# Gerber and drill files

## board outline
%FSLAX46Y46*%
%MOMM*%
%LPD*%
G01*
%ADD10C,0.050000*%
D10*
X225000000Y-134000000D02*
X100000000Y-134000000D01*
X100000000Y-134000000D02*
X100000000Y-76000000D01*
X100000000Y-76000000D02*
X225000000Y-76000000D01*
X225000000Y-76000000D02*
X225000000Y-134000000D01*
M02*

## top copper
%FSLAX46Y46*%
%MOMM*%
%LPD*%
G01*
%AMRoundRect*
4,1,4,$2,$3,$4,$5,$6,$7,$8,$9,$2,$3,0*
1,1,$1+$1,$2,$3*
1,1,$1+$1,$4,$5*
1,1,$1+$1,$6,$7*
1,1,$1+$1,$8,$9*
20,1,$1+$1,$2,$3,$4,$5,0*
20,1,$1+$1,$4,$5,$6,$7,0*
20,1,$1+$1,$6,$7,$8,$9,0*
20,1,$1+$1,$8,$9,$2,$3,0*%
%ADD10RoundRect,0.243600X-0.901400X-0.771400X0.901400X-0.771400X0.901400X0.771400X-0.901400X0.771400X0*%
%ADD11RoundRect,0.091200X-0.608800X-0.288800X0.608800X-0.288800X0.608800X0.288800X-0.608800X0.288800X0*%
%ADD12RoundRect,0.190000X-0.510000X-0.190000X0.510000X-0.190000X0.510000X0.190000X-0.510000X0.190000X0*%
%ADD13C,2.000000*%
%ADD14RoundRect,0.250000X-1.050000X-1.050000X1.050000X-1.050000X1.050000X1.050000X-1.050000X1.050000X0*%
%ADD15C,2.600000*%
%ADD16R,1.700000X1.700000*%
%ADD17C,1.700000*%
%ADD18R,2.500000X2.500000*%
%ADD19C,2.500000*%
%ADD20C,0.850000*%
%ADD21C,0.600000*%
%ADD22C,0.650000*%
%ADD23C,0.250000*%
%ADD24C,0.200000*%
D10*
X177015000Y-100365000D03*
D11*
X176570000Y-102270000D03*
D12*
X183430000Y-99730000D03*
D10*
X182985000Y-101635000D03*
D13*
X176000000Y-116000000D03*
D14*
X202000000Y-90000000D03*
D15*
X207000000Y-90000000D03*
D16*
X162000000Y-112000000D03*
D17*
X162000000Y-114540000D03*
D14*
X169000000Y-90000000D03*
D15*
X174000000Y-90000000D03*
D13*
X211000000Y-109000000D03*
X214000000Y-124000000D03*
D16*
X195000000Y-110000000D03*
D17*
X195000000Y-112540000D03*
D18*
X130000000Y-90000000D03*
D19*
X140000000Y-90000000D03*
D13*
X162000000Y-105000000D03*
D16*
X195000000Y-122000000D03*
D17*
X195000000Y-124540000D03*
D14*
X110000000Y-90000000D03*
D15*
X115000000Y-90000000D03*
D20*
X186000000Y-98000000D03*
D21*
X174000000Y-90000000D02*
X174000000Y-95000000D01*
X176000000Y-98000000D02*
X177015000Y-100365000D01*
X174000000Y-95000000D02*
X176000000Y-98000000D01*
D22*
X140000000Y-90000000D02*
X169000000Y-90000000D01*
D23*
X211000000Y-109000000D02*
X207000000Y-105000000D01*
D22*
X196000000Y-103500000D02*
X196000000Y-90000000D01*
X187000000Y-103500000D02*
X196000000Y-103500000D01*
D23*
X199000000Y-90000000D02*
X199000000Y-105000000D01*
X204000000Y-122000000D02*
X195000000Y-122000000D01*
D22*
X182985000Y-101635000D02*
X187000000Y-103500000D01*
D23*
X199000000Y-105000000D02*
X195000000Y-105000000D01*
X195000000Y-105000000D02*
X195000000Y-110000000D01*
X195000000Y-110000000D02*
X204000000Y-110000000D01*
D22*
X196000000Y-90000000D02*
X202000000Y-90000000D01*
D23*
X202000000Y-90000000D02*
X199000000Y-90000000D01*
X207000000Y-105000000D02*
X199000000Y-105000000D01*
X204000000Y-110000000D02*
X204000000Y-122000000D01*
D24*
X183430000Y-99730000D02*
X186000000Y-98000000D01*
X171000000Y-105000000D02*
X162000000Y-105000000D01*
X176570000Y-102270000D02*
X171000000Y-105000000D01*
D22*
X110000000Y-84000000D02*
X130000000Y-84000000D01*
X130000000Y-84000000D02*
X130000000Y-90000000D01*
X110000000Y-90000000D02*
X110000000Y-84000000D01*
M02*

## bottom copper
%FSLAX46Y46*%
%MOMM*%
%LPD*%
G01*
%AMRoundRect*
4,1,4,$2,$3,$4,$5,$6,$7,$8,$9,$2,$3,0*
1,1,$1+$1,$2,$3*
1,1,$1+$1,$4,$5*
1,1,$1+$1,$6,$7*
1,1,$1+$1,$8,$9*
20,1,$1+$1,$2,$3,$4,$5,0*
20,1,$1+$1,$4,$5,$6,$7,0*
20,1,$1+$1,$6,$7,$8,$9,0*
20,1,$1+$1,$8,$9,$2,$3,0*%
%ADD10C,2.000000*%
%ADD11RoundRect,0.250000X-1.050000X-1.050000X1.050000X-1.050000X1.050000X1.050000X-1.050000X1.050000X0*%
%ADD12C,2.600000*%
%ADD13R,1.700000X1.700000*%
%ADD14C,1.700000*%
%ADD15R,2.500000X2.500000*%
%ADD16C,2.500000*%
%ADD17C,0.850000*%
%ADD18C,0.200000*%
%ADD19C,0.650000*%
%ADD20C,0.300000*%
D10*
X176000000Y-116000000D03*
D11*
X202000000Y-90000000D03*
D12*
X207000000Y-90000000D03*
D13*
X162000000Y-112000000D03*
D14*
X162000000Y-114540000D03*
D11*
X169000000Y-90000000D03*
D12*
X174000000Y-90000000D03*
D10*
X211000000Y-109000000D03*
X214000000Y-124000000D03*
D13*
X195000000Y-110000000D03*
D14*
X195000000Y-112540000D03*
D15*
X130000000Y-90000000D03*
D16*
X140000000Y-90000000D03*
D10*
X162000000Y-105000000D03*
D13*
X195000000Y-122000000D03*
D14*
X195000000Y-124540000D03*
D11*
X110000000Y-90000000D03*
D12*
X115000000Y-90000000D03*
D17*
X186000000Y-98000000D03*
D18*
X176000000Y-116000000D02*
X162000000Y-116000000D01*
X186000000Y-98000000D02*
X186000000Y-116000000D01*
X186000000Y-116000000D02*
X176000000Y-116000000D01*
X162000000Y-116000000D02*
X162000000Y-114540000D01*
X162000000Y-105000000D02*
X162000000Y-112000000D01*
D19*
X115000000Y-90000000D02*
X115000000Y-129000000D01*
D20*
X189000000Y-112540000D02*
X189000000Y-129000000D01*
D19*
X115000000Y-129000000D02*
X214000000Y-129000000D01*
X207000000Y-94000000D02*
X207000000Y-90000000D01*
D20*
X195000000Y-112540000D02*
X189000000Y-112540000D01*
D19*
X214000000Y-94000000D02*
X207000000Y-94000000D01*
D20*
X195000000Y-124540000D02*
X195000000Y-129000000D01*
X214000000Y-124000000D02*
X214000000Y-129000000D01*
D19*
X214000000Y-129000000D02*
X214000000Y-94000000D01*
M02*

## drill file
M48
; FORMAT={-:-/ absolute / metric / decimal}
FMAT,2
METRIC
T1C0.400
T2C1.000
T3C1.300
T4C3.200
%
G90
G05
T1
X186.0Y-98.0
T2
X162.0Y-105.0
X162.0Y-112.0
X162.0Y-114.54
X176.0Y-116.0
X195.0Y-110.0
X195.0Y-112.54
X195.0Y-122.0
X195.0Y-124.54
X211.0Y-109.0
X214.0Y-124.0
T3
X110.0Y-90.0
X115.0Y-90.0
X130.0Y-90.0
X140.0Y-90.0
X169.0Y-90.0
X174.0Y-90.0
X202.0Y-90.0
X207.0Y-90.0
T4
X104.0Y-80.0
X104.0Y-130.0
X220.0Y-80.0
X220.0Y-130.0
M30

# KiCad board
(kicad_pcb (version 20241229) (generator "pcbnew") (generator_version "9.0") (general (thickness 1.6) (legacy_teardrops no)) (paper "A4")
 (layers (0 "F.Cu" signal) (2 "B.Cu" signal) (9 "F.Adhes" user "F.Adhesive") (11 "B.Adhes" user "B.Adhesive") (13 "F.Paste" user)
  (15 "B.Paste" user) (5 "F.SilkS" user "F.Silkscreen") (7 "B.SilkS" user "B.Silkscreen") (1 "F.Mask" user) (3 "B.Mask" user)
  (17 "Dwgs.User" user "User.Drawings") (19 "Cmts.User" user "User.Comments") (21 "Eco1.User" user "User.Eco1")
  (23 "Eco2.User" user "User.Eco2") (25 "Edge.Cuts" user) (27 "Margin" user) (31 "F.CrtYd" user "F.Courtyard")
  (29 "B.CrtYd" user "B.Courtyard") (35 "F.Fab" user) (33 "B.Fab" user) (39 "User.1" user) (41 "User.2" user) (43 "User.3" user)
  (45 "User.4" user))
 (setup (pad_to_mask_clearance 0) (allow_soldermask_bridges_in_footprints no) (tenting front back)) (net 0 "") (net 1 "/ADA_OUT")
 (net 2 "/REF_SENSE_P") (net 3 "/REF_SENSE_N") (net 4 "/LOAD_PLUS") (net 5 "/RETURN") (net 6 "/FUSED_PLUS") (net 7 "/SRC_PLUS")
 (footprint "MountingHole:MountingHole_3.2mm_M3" (layer "F.Cu") (at 220 130)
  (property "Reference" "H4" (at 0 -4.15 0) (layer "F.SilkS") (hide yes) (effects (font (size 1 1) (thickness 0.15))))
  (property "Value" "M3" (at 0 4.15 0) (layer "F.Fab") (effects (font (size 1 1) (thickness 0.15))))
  (pad "" np_thru_hole circle (at 0 0) (size 3.2 3.2) (drill 3.2) (layers "*.Cu" "*.Mask")))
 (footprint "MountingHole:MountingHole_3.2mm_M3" (layer "F.Cu") (at 104 80)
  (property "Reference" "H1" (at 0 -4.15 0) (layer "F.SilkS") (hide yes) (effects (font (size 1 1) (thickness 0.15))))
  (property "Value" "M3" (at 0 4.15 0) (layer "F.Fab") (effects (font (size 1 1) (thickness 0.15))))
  (pad "" np_thru_hole circle (at 0 0) (size 3.2 3.2) (drill 3.2) (layers "*.Cu" "*.Mask")))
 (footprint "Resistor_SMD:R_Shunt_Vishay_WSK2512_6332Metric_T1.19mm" (layer "F.Cu") (at 180 101)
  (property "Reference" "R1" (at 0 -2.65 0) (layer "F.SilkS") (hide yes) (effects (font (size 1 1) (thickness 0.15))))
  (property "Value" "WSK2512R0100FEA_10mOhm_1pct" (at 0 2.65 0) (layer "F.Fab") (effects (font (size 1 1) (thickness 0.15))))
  (pad "1" smd roundrect (at -2.985 -0.635) (size 2.29 2.03) (layers "F.Cu" "F.Mask" "F.Paste") (roundrect_rratio 0.12) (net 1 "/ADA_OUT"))
  (pad "2" smd roundrect (at -3.43 1.27) (size 1.4 0.76) (layers "F.Cu" "F.Mask" "F.Paste") (roundrect_rratio 0.12) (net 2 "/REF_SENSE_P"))
  (pad "3" smd roundrect (at 3.43 -1.27) (size 1.4 0.76) (layers "F.Cu" "F.Mask" "F.Paste") (roundrect_rratio 0.25) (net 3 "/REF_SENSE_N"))
  (pad "4" smd roundrect (at 2.985 0.635) (size 2.29 2.03) (layers "F.Cu" "F.Mask" "F.Paste") (roundrect_rratio 0.12) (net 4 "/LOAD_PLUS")))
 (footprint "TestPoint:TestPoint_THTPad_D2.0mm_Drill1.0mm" (layer "F.Cu") (at 176 116)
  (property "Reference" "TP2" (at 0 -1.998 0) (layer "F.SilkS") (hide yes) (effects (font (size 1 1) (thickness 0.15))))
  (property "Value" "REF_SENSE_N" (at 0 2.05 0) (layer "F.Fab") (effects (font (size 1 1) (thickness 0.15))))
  (pad "1" thru_hole circle (at 0 0) (size 2 2) (drill 1) (layers "*.Cu" "*.Mask") (remove_unused_layers no) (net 3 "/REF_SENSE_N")))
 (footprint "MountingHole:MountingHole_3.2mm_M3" (layer "F.Cu") (at 220 80)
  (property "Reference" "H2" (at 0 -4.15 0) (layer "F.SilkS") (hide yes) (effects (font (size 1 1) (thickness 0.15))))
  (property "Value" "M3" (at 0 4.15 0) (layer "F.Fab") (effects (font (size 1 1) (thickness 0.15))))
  (pad "" np_thru_hole circle (at 0 0) (size 3.2 3.2) (drill 3.2) (layers "*.Cu" "*.Mask")))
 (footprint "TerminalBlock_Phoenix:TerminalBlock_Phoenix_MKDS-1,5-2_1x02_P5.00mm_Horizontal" (layer "F.Cu") (at 202 90)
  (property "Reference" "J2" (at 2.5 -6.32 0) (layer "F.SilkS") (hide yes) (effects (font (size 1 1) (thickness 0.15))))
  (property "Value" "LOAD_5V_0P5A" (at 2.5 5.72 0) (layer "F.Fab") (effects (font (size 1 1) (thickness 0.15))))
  (pad "1" thru_hole roundrect (at 0 0) (size 2.6 2.6) (drill 1.3) (layers "*.Cu" "*.Mask") (remove_unused_layers no)
   (roundrect_rratio 0.096154) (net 4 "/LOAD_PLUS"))
  (pad "2" thru_hole circle (at 5 0) (size 2.6 2.6) (drill 1.3) (layers "*.Cu" "*.Mask") (remove_unused_layers no) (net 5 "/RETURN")))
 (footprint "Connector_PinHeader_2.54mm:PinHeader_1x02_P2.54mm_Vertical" (layer "F.Cu") (at 162 112)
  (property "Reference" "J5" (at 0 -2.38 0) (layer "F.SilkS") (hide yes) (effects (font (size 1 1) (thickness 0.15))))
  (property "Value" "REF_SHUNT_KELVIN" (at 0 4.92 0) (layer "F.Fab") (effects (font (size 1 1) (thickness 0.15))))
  (pad "1" thru_hole rect (at 0 0) (size 1.7 1.7) (drill 1) (layers "*.Cu" "*.Mask") (remove_unused_layers no) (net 2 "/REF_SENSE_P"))
  (pad "2" thru_hole circle (at 0 2.54) (size 1.7 1.7) (drill 1) (layers "*.Cu" "*.Mask") (remove_unused_layers no) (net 3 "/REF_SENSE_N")))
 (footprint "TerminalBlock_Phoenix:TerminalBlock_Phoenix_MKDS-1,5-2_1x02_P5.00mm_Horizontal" (layer "F.Cu") (at 169 90)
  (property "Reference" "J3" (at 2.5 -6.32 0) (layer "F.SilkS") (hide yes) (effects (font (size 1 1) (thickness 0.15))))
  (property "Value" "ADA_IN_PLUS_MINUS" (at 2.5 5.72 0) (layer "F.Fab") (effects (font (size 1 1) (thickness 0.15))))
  (pad "1" thru_hole roundrect (at 0 0) (size 2.6 2.6) (drill 1.3) (layers "*.Cu" "*.Mask") (remove_unused_layers no)
   (roundrect_rratio 0.096154) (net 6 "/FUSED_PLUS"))
  (pad "2" thru_hole circle (at 5 0) (size 2.6 2.6) (drill 1.3) (layers "*.Cu" "*.Mask") (remove_unused_layers no) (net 1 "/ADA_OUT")))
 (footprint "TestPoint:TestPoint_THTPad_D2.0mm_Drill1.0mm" (layer "F.Cu") (at 211 109)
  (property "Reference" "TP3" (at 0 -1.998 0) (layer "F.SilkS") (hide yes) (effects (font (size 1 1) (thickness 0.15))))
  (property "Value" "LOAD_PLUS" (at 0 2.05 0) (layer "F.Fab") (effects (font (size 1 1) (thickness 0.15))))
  (pad "1" thru_hole circle (at 0 0) (size 2 2) (drill 1) (layers "*.Cu" "*.Mask") (remove_unused_layers no) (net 4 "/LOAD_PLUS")))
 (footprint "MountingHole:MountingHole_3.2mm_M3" (layer "F.Cu") (at 104 130)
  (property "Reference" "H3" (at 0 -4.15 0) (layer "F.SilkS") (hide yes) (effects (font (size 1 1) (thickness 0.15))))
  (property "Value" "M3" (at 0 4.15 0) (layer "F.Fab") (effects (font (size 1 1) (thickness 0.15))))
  (pad "" np_thru_hole circle (at 0 0) (size 3.2 3.2) (drill 3.2) (layers "*.Cu" "*.Mask")))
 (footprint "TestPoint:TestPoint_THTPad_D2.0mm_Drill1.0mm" (layer "F.Cu") (at 214 124)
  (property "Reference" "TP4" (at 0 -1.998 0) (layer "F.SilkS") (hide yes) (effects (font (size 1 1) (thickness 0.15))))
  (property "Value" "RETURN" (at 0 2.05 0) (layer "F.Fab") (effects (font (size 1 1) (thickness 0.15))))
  (pad "1" thru_hole circle (at 0 0) (size 2 2) (drill 1) (layers "*.Cu" "*.Mask") (remove_unused_layers no) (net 5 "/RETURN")))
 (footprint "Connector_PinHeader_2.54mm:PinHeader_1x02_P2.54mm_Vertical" (layer "F.Cu") (at 195 110)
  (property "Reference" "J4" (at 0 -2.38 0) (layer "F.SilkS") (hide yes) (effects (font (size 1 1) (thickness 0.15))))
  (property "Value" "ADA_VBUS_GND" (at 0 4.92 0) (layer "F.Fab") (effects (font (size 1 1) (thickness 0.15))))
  (pad "1" thru_hole rect (at 0 0) (size 1.7 1.7) (drill 1) (layers "*.Cu" "*.Mask") (remove_unused_layers no) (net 4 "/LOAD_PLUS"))
  (pad "2" thru_hole circle (at 0 2.54) (size 1.7 1.7) (drill 1) (layers "*.Cu" "*.Mask") (remove_unused_layers no) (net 5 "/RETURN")))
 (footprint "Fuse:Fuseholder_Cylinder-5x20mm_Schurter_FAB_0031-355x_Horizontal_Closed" (layer "F.Cu") (at 130 90)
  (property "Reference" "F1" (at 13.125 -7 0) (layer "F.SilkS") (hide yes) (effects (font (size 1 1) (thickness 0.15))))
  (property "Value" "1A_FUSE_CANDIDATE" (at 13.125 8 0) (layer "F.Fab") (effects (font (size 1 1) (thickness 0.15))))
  (pad "1" thru_hole rect (at 0 0) (size 2.5 2.5) (drill 1.3) (layers "*.Cu" "*.Mask") (remove_unused_layers no) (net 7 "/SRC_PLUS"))
  (pad "2" thru_hole circle (at 10 0) (size 2.5 2.5) (drill 1.3) (layers "*.Cu" "*.Mask") (remove_unused_layers no) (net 6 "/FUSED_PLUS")))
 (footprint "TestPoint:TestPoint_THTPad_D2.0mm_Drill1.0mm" (layer "F.Cu") (at 162 105)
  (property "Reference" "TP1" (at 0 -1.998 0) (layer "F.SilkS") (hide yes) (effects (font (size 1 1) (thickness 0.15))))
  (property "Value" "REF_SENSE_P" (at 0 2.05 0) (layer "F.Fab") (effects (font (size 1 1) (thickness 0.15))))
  (pad "1" thru_hole circle (at 0 0) (size 2 2) (drill 1) (layers "*.Cu" "*.Mask") (remove_unused_layers no) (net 2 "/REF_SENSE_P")))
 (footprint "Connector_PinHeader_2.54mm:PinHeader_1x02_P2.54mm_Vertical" (layer "F.Cu") (at 195 122)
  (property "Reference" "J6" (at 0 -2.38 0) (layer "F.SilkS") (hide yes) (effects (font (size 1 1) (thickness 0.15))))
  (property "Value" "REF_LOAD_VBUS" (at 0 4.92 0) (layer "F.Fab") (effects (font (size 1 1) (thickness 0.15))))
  (pad "1" thru_hole rect (at 0 0) (size 1.7 1.7) (drill 1) (layers "*.Cu" "*.Mask") (remove_unused_layers no) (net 4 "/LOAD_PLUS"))
  (pad "2" thru_hole circle (at 0 2.54) (size 1.7 1.7) (drill 1) (layers "*.Cu" "*.Mask") (remove_unused_layers no) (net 5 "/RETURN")))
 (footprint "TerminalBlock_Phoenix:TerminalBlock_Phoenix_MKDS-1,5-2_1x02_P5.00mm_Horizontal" (layer "F.Cu") (at 110 90)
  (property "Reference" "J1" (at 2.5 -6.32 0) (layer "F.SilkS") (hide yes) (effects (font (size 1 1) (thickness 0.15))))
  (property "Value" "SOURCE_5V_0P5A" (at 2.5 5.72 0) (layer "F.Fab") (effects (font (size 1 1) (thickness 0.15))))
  (pad "1" thru_hole roundrect (at 0 0) (size 2.6 2.6) (drill 1.3) (layers "*.Cu" "*.Mask") (remove_unused_layers no)
   (roundrect_rratio 0.096154) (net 7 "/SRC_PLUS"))
  (pad "2" thru_hole circle (at 5 0) (size 2.6 2.6) (drill 1.3) (layers "*.Cu" "*.Mask") (remove_unused_layers no) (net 5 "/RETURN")))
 (gr_line (start 225 134) (end 100 134) (stroke (width 0.05) (type default)) (layer "Edge.Cuts"))
 (gr_line (start 100 134) (end 100 76) (stroke (width 0.05) (type default)) (layer "Edge.Cuts"))
 (gr_line (start 100 76) (end 225 76) (stroke (width 0.05) (type default)) (layer "Edge.Cuts"))
 (gr_line (start 225 76) (end 225 134) (stroke (width 0.05) (type default)) (layer "Edge.Cuts"))
 (segment (start 174 90) (end 174 95) (width 0.6) (layer "F.Cu") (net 1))
 (segment (start 176 98) (end 177.015 100.365) (width 0.6) (layer "F.Cu") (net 1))
 (segment (start 174 95) (end 176 98) (width 0.6) (layer "F.Cu") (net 1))
 (segment (start 140 90) (end 169 90) (width 0.65) (layer "F.Cu") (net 6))
 (segment (start 211 109) (end 207 105) (width 0.25) (layer "F.Cu") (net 4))
 (segment (start 196 103.5) (end 196 90) (width 0.65) (layer "F.Cu") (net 4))
 (segment (start 187 103.5) (end 196 103.5) (width 0.65) (layer "F.Cu") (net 4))
 (segment (start 199 90) (end 199 105) (width 0.25) (layer "F.Cu") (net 4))
 (segment (start 204 122) (end 195 122) (width 0.25) (layer "F.Cu") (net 4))
 (segment (start 182.985 101.635) (end 187 103.5) (width 0.65) (layer "F.Cu") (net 4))
 (segment (start 199 105) (end 195 105) (width 0.25) (layer "F.Cu") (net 4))
 (segment (start 195 105) (end 195 110) (width 0.25) (layer "F.Cu") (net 4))
 (segment (start 195 110) (end 204 110) (width 0.25) (layer "F.Cu") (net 4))
 (segment (start 196 90) (end 202 90) (width 0.65) (layer "F.Cu") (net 4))
 (segment (start 202 90) (end 199 90) (width 0.25) (layer "F.Cu") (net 4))
 (segment (start 207 105) (end 199 105) (width 0.25) (layer "F.Cu") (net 4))
 (segment (start 204 110) (end 204 122) (width 0.25) (layer "F.Cu") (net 4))
 (segment (start 183.43 99.73) (end 186 98) (width 0.2) (layer "F.Cu") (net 3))
 (via (at 186 98) (size 0.85) (drill 0.4) (layers "F.Cu" "B.Cu") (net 3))
 (segment (start 176 116) (end 162 116) (width 0.2) (layer "B.Cu") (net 3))
 (segment (start 186 98) (end 186 116) (width 0.2) (layer "B.Cu") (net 3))
 (segment (start 186 116) (end 176 116) (width 0.2) (layer "B.Cu") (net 3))
 (segment (start 162 116) (end 162 114.54) (width 0.2) (layer "B.Cu") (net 3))
 (segment (start 171 105) (end 162 105) (width 0.2) (layer "F.Cu") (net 2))
 (segment (start 176.57 102.27) (end 171 105) (width 0.2) (layer "F.Cu") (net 2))
 (segment (start 162 105) (end 162 112) (width 0.2) (layer "B.Cu") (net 2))
 (segment (start 115 90) (end 115 129) (width 0.65) (layer "B.Cu") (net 5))
 (segment (start 189 112.54) (end 189 129) (width 0.3) (layer "B.Cu") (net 5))
 (segment (start 115 129) (end 214 129) (width 0.65) (layer "B.Cu") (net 5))
 (segment (start 207 94) (end 207 90) (width 0.65) (layer "B.Cu") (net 5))
 (segment (start 195 112.54) (end 189 112.54) (width 0.3) (layer "B.Cu") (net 5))
 (segment (start 214 94) (end 207 94) (width 0.65) (layer "B.Cu") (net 5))
 (segment (start 195 124.54) (end 195 129) (width 0.3) (layer "B.Cu") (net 5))
 (segment (start 214 124) (end 214 129) (width 0.3) (layer "B.Cu") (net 5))
 (segment (start 214 129) (end 214 94) (width 0.65) (layer "B.Cu") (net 5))
 (segment (start 110 84) (end 130 84) (width 0.65) (layer "F.Cu") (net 7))
 (segment (start 130 84) (end 130 90) (width 0.65) (layer "F.Cu") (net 7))
 (segment (start 110 90) (end 110 84) (width 0.65) (layer "F.Cu") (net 7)))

